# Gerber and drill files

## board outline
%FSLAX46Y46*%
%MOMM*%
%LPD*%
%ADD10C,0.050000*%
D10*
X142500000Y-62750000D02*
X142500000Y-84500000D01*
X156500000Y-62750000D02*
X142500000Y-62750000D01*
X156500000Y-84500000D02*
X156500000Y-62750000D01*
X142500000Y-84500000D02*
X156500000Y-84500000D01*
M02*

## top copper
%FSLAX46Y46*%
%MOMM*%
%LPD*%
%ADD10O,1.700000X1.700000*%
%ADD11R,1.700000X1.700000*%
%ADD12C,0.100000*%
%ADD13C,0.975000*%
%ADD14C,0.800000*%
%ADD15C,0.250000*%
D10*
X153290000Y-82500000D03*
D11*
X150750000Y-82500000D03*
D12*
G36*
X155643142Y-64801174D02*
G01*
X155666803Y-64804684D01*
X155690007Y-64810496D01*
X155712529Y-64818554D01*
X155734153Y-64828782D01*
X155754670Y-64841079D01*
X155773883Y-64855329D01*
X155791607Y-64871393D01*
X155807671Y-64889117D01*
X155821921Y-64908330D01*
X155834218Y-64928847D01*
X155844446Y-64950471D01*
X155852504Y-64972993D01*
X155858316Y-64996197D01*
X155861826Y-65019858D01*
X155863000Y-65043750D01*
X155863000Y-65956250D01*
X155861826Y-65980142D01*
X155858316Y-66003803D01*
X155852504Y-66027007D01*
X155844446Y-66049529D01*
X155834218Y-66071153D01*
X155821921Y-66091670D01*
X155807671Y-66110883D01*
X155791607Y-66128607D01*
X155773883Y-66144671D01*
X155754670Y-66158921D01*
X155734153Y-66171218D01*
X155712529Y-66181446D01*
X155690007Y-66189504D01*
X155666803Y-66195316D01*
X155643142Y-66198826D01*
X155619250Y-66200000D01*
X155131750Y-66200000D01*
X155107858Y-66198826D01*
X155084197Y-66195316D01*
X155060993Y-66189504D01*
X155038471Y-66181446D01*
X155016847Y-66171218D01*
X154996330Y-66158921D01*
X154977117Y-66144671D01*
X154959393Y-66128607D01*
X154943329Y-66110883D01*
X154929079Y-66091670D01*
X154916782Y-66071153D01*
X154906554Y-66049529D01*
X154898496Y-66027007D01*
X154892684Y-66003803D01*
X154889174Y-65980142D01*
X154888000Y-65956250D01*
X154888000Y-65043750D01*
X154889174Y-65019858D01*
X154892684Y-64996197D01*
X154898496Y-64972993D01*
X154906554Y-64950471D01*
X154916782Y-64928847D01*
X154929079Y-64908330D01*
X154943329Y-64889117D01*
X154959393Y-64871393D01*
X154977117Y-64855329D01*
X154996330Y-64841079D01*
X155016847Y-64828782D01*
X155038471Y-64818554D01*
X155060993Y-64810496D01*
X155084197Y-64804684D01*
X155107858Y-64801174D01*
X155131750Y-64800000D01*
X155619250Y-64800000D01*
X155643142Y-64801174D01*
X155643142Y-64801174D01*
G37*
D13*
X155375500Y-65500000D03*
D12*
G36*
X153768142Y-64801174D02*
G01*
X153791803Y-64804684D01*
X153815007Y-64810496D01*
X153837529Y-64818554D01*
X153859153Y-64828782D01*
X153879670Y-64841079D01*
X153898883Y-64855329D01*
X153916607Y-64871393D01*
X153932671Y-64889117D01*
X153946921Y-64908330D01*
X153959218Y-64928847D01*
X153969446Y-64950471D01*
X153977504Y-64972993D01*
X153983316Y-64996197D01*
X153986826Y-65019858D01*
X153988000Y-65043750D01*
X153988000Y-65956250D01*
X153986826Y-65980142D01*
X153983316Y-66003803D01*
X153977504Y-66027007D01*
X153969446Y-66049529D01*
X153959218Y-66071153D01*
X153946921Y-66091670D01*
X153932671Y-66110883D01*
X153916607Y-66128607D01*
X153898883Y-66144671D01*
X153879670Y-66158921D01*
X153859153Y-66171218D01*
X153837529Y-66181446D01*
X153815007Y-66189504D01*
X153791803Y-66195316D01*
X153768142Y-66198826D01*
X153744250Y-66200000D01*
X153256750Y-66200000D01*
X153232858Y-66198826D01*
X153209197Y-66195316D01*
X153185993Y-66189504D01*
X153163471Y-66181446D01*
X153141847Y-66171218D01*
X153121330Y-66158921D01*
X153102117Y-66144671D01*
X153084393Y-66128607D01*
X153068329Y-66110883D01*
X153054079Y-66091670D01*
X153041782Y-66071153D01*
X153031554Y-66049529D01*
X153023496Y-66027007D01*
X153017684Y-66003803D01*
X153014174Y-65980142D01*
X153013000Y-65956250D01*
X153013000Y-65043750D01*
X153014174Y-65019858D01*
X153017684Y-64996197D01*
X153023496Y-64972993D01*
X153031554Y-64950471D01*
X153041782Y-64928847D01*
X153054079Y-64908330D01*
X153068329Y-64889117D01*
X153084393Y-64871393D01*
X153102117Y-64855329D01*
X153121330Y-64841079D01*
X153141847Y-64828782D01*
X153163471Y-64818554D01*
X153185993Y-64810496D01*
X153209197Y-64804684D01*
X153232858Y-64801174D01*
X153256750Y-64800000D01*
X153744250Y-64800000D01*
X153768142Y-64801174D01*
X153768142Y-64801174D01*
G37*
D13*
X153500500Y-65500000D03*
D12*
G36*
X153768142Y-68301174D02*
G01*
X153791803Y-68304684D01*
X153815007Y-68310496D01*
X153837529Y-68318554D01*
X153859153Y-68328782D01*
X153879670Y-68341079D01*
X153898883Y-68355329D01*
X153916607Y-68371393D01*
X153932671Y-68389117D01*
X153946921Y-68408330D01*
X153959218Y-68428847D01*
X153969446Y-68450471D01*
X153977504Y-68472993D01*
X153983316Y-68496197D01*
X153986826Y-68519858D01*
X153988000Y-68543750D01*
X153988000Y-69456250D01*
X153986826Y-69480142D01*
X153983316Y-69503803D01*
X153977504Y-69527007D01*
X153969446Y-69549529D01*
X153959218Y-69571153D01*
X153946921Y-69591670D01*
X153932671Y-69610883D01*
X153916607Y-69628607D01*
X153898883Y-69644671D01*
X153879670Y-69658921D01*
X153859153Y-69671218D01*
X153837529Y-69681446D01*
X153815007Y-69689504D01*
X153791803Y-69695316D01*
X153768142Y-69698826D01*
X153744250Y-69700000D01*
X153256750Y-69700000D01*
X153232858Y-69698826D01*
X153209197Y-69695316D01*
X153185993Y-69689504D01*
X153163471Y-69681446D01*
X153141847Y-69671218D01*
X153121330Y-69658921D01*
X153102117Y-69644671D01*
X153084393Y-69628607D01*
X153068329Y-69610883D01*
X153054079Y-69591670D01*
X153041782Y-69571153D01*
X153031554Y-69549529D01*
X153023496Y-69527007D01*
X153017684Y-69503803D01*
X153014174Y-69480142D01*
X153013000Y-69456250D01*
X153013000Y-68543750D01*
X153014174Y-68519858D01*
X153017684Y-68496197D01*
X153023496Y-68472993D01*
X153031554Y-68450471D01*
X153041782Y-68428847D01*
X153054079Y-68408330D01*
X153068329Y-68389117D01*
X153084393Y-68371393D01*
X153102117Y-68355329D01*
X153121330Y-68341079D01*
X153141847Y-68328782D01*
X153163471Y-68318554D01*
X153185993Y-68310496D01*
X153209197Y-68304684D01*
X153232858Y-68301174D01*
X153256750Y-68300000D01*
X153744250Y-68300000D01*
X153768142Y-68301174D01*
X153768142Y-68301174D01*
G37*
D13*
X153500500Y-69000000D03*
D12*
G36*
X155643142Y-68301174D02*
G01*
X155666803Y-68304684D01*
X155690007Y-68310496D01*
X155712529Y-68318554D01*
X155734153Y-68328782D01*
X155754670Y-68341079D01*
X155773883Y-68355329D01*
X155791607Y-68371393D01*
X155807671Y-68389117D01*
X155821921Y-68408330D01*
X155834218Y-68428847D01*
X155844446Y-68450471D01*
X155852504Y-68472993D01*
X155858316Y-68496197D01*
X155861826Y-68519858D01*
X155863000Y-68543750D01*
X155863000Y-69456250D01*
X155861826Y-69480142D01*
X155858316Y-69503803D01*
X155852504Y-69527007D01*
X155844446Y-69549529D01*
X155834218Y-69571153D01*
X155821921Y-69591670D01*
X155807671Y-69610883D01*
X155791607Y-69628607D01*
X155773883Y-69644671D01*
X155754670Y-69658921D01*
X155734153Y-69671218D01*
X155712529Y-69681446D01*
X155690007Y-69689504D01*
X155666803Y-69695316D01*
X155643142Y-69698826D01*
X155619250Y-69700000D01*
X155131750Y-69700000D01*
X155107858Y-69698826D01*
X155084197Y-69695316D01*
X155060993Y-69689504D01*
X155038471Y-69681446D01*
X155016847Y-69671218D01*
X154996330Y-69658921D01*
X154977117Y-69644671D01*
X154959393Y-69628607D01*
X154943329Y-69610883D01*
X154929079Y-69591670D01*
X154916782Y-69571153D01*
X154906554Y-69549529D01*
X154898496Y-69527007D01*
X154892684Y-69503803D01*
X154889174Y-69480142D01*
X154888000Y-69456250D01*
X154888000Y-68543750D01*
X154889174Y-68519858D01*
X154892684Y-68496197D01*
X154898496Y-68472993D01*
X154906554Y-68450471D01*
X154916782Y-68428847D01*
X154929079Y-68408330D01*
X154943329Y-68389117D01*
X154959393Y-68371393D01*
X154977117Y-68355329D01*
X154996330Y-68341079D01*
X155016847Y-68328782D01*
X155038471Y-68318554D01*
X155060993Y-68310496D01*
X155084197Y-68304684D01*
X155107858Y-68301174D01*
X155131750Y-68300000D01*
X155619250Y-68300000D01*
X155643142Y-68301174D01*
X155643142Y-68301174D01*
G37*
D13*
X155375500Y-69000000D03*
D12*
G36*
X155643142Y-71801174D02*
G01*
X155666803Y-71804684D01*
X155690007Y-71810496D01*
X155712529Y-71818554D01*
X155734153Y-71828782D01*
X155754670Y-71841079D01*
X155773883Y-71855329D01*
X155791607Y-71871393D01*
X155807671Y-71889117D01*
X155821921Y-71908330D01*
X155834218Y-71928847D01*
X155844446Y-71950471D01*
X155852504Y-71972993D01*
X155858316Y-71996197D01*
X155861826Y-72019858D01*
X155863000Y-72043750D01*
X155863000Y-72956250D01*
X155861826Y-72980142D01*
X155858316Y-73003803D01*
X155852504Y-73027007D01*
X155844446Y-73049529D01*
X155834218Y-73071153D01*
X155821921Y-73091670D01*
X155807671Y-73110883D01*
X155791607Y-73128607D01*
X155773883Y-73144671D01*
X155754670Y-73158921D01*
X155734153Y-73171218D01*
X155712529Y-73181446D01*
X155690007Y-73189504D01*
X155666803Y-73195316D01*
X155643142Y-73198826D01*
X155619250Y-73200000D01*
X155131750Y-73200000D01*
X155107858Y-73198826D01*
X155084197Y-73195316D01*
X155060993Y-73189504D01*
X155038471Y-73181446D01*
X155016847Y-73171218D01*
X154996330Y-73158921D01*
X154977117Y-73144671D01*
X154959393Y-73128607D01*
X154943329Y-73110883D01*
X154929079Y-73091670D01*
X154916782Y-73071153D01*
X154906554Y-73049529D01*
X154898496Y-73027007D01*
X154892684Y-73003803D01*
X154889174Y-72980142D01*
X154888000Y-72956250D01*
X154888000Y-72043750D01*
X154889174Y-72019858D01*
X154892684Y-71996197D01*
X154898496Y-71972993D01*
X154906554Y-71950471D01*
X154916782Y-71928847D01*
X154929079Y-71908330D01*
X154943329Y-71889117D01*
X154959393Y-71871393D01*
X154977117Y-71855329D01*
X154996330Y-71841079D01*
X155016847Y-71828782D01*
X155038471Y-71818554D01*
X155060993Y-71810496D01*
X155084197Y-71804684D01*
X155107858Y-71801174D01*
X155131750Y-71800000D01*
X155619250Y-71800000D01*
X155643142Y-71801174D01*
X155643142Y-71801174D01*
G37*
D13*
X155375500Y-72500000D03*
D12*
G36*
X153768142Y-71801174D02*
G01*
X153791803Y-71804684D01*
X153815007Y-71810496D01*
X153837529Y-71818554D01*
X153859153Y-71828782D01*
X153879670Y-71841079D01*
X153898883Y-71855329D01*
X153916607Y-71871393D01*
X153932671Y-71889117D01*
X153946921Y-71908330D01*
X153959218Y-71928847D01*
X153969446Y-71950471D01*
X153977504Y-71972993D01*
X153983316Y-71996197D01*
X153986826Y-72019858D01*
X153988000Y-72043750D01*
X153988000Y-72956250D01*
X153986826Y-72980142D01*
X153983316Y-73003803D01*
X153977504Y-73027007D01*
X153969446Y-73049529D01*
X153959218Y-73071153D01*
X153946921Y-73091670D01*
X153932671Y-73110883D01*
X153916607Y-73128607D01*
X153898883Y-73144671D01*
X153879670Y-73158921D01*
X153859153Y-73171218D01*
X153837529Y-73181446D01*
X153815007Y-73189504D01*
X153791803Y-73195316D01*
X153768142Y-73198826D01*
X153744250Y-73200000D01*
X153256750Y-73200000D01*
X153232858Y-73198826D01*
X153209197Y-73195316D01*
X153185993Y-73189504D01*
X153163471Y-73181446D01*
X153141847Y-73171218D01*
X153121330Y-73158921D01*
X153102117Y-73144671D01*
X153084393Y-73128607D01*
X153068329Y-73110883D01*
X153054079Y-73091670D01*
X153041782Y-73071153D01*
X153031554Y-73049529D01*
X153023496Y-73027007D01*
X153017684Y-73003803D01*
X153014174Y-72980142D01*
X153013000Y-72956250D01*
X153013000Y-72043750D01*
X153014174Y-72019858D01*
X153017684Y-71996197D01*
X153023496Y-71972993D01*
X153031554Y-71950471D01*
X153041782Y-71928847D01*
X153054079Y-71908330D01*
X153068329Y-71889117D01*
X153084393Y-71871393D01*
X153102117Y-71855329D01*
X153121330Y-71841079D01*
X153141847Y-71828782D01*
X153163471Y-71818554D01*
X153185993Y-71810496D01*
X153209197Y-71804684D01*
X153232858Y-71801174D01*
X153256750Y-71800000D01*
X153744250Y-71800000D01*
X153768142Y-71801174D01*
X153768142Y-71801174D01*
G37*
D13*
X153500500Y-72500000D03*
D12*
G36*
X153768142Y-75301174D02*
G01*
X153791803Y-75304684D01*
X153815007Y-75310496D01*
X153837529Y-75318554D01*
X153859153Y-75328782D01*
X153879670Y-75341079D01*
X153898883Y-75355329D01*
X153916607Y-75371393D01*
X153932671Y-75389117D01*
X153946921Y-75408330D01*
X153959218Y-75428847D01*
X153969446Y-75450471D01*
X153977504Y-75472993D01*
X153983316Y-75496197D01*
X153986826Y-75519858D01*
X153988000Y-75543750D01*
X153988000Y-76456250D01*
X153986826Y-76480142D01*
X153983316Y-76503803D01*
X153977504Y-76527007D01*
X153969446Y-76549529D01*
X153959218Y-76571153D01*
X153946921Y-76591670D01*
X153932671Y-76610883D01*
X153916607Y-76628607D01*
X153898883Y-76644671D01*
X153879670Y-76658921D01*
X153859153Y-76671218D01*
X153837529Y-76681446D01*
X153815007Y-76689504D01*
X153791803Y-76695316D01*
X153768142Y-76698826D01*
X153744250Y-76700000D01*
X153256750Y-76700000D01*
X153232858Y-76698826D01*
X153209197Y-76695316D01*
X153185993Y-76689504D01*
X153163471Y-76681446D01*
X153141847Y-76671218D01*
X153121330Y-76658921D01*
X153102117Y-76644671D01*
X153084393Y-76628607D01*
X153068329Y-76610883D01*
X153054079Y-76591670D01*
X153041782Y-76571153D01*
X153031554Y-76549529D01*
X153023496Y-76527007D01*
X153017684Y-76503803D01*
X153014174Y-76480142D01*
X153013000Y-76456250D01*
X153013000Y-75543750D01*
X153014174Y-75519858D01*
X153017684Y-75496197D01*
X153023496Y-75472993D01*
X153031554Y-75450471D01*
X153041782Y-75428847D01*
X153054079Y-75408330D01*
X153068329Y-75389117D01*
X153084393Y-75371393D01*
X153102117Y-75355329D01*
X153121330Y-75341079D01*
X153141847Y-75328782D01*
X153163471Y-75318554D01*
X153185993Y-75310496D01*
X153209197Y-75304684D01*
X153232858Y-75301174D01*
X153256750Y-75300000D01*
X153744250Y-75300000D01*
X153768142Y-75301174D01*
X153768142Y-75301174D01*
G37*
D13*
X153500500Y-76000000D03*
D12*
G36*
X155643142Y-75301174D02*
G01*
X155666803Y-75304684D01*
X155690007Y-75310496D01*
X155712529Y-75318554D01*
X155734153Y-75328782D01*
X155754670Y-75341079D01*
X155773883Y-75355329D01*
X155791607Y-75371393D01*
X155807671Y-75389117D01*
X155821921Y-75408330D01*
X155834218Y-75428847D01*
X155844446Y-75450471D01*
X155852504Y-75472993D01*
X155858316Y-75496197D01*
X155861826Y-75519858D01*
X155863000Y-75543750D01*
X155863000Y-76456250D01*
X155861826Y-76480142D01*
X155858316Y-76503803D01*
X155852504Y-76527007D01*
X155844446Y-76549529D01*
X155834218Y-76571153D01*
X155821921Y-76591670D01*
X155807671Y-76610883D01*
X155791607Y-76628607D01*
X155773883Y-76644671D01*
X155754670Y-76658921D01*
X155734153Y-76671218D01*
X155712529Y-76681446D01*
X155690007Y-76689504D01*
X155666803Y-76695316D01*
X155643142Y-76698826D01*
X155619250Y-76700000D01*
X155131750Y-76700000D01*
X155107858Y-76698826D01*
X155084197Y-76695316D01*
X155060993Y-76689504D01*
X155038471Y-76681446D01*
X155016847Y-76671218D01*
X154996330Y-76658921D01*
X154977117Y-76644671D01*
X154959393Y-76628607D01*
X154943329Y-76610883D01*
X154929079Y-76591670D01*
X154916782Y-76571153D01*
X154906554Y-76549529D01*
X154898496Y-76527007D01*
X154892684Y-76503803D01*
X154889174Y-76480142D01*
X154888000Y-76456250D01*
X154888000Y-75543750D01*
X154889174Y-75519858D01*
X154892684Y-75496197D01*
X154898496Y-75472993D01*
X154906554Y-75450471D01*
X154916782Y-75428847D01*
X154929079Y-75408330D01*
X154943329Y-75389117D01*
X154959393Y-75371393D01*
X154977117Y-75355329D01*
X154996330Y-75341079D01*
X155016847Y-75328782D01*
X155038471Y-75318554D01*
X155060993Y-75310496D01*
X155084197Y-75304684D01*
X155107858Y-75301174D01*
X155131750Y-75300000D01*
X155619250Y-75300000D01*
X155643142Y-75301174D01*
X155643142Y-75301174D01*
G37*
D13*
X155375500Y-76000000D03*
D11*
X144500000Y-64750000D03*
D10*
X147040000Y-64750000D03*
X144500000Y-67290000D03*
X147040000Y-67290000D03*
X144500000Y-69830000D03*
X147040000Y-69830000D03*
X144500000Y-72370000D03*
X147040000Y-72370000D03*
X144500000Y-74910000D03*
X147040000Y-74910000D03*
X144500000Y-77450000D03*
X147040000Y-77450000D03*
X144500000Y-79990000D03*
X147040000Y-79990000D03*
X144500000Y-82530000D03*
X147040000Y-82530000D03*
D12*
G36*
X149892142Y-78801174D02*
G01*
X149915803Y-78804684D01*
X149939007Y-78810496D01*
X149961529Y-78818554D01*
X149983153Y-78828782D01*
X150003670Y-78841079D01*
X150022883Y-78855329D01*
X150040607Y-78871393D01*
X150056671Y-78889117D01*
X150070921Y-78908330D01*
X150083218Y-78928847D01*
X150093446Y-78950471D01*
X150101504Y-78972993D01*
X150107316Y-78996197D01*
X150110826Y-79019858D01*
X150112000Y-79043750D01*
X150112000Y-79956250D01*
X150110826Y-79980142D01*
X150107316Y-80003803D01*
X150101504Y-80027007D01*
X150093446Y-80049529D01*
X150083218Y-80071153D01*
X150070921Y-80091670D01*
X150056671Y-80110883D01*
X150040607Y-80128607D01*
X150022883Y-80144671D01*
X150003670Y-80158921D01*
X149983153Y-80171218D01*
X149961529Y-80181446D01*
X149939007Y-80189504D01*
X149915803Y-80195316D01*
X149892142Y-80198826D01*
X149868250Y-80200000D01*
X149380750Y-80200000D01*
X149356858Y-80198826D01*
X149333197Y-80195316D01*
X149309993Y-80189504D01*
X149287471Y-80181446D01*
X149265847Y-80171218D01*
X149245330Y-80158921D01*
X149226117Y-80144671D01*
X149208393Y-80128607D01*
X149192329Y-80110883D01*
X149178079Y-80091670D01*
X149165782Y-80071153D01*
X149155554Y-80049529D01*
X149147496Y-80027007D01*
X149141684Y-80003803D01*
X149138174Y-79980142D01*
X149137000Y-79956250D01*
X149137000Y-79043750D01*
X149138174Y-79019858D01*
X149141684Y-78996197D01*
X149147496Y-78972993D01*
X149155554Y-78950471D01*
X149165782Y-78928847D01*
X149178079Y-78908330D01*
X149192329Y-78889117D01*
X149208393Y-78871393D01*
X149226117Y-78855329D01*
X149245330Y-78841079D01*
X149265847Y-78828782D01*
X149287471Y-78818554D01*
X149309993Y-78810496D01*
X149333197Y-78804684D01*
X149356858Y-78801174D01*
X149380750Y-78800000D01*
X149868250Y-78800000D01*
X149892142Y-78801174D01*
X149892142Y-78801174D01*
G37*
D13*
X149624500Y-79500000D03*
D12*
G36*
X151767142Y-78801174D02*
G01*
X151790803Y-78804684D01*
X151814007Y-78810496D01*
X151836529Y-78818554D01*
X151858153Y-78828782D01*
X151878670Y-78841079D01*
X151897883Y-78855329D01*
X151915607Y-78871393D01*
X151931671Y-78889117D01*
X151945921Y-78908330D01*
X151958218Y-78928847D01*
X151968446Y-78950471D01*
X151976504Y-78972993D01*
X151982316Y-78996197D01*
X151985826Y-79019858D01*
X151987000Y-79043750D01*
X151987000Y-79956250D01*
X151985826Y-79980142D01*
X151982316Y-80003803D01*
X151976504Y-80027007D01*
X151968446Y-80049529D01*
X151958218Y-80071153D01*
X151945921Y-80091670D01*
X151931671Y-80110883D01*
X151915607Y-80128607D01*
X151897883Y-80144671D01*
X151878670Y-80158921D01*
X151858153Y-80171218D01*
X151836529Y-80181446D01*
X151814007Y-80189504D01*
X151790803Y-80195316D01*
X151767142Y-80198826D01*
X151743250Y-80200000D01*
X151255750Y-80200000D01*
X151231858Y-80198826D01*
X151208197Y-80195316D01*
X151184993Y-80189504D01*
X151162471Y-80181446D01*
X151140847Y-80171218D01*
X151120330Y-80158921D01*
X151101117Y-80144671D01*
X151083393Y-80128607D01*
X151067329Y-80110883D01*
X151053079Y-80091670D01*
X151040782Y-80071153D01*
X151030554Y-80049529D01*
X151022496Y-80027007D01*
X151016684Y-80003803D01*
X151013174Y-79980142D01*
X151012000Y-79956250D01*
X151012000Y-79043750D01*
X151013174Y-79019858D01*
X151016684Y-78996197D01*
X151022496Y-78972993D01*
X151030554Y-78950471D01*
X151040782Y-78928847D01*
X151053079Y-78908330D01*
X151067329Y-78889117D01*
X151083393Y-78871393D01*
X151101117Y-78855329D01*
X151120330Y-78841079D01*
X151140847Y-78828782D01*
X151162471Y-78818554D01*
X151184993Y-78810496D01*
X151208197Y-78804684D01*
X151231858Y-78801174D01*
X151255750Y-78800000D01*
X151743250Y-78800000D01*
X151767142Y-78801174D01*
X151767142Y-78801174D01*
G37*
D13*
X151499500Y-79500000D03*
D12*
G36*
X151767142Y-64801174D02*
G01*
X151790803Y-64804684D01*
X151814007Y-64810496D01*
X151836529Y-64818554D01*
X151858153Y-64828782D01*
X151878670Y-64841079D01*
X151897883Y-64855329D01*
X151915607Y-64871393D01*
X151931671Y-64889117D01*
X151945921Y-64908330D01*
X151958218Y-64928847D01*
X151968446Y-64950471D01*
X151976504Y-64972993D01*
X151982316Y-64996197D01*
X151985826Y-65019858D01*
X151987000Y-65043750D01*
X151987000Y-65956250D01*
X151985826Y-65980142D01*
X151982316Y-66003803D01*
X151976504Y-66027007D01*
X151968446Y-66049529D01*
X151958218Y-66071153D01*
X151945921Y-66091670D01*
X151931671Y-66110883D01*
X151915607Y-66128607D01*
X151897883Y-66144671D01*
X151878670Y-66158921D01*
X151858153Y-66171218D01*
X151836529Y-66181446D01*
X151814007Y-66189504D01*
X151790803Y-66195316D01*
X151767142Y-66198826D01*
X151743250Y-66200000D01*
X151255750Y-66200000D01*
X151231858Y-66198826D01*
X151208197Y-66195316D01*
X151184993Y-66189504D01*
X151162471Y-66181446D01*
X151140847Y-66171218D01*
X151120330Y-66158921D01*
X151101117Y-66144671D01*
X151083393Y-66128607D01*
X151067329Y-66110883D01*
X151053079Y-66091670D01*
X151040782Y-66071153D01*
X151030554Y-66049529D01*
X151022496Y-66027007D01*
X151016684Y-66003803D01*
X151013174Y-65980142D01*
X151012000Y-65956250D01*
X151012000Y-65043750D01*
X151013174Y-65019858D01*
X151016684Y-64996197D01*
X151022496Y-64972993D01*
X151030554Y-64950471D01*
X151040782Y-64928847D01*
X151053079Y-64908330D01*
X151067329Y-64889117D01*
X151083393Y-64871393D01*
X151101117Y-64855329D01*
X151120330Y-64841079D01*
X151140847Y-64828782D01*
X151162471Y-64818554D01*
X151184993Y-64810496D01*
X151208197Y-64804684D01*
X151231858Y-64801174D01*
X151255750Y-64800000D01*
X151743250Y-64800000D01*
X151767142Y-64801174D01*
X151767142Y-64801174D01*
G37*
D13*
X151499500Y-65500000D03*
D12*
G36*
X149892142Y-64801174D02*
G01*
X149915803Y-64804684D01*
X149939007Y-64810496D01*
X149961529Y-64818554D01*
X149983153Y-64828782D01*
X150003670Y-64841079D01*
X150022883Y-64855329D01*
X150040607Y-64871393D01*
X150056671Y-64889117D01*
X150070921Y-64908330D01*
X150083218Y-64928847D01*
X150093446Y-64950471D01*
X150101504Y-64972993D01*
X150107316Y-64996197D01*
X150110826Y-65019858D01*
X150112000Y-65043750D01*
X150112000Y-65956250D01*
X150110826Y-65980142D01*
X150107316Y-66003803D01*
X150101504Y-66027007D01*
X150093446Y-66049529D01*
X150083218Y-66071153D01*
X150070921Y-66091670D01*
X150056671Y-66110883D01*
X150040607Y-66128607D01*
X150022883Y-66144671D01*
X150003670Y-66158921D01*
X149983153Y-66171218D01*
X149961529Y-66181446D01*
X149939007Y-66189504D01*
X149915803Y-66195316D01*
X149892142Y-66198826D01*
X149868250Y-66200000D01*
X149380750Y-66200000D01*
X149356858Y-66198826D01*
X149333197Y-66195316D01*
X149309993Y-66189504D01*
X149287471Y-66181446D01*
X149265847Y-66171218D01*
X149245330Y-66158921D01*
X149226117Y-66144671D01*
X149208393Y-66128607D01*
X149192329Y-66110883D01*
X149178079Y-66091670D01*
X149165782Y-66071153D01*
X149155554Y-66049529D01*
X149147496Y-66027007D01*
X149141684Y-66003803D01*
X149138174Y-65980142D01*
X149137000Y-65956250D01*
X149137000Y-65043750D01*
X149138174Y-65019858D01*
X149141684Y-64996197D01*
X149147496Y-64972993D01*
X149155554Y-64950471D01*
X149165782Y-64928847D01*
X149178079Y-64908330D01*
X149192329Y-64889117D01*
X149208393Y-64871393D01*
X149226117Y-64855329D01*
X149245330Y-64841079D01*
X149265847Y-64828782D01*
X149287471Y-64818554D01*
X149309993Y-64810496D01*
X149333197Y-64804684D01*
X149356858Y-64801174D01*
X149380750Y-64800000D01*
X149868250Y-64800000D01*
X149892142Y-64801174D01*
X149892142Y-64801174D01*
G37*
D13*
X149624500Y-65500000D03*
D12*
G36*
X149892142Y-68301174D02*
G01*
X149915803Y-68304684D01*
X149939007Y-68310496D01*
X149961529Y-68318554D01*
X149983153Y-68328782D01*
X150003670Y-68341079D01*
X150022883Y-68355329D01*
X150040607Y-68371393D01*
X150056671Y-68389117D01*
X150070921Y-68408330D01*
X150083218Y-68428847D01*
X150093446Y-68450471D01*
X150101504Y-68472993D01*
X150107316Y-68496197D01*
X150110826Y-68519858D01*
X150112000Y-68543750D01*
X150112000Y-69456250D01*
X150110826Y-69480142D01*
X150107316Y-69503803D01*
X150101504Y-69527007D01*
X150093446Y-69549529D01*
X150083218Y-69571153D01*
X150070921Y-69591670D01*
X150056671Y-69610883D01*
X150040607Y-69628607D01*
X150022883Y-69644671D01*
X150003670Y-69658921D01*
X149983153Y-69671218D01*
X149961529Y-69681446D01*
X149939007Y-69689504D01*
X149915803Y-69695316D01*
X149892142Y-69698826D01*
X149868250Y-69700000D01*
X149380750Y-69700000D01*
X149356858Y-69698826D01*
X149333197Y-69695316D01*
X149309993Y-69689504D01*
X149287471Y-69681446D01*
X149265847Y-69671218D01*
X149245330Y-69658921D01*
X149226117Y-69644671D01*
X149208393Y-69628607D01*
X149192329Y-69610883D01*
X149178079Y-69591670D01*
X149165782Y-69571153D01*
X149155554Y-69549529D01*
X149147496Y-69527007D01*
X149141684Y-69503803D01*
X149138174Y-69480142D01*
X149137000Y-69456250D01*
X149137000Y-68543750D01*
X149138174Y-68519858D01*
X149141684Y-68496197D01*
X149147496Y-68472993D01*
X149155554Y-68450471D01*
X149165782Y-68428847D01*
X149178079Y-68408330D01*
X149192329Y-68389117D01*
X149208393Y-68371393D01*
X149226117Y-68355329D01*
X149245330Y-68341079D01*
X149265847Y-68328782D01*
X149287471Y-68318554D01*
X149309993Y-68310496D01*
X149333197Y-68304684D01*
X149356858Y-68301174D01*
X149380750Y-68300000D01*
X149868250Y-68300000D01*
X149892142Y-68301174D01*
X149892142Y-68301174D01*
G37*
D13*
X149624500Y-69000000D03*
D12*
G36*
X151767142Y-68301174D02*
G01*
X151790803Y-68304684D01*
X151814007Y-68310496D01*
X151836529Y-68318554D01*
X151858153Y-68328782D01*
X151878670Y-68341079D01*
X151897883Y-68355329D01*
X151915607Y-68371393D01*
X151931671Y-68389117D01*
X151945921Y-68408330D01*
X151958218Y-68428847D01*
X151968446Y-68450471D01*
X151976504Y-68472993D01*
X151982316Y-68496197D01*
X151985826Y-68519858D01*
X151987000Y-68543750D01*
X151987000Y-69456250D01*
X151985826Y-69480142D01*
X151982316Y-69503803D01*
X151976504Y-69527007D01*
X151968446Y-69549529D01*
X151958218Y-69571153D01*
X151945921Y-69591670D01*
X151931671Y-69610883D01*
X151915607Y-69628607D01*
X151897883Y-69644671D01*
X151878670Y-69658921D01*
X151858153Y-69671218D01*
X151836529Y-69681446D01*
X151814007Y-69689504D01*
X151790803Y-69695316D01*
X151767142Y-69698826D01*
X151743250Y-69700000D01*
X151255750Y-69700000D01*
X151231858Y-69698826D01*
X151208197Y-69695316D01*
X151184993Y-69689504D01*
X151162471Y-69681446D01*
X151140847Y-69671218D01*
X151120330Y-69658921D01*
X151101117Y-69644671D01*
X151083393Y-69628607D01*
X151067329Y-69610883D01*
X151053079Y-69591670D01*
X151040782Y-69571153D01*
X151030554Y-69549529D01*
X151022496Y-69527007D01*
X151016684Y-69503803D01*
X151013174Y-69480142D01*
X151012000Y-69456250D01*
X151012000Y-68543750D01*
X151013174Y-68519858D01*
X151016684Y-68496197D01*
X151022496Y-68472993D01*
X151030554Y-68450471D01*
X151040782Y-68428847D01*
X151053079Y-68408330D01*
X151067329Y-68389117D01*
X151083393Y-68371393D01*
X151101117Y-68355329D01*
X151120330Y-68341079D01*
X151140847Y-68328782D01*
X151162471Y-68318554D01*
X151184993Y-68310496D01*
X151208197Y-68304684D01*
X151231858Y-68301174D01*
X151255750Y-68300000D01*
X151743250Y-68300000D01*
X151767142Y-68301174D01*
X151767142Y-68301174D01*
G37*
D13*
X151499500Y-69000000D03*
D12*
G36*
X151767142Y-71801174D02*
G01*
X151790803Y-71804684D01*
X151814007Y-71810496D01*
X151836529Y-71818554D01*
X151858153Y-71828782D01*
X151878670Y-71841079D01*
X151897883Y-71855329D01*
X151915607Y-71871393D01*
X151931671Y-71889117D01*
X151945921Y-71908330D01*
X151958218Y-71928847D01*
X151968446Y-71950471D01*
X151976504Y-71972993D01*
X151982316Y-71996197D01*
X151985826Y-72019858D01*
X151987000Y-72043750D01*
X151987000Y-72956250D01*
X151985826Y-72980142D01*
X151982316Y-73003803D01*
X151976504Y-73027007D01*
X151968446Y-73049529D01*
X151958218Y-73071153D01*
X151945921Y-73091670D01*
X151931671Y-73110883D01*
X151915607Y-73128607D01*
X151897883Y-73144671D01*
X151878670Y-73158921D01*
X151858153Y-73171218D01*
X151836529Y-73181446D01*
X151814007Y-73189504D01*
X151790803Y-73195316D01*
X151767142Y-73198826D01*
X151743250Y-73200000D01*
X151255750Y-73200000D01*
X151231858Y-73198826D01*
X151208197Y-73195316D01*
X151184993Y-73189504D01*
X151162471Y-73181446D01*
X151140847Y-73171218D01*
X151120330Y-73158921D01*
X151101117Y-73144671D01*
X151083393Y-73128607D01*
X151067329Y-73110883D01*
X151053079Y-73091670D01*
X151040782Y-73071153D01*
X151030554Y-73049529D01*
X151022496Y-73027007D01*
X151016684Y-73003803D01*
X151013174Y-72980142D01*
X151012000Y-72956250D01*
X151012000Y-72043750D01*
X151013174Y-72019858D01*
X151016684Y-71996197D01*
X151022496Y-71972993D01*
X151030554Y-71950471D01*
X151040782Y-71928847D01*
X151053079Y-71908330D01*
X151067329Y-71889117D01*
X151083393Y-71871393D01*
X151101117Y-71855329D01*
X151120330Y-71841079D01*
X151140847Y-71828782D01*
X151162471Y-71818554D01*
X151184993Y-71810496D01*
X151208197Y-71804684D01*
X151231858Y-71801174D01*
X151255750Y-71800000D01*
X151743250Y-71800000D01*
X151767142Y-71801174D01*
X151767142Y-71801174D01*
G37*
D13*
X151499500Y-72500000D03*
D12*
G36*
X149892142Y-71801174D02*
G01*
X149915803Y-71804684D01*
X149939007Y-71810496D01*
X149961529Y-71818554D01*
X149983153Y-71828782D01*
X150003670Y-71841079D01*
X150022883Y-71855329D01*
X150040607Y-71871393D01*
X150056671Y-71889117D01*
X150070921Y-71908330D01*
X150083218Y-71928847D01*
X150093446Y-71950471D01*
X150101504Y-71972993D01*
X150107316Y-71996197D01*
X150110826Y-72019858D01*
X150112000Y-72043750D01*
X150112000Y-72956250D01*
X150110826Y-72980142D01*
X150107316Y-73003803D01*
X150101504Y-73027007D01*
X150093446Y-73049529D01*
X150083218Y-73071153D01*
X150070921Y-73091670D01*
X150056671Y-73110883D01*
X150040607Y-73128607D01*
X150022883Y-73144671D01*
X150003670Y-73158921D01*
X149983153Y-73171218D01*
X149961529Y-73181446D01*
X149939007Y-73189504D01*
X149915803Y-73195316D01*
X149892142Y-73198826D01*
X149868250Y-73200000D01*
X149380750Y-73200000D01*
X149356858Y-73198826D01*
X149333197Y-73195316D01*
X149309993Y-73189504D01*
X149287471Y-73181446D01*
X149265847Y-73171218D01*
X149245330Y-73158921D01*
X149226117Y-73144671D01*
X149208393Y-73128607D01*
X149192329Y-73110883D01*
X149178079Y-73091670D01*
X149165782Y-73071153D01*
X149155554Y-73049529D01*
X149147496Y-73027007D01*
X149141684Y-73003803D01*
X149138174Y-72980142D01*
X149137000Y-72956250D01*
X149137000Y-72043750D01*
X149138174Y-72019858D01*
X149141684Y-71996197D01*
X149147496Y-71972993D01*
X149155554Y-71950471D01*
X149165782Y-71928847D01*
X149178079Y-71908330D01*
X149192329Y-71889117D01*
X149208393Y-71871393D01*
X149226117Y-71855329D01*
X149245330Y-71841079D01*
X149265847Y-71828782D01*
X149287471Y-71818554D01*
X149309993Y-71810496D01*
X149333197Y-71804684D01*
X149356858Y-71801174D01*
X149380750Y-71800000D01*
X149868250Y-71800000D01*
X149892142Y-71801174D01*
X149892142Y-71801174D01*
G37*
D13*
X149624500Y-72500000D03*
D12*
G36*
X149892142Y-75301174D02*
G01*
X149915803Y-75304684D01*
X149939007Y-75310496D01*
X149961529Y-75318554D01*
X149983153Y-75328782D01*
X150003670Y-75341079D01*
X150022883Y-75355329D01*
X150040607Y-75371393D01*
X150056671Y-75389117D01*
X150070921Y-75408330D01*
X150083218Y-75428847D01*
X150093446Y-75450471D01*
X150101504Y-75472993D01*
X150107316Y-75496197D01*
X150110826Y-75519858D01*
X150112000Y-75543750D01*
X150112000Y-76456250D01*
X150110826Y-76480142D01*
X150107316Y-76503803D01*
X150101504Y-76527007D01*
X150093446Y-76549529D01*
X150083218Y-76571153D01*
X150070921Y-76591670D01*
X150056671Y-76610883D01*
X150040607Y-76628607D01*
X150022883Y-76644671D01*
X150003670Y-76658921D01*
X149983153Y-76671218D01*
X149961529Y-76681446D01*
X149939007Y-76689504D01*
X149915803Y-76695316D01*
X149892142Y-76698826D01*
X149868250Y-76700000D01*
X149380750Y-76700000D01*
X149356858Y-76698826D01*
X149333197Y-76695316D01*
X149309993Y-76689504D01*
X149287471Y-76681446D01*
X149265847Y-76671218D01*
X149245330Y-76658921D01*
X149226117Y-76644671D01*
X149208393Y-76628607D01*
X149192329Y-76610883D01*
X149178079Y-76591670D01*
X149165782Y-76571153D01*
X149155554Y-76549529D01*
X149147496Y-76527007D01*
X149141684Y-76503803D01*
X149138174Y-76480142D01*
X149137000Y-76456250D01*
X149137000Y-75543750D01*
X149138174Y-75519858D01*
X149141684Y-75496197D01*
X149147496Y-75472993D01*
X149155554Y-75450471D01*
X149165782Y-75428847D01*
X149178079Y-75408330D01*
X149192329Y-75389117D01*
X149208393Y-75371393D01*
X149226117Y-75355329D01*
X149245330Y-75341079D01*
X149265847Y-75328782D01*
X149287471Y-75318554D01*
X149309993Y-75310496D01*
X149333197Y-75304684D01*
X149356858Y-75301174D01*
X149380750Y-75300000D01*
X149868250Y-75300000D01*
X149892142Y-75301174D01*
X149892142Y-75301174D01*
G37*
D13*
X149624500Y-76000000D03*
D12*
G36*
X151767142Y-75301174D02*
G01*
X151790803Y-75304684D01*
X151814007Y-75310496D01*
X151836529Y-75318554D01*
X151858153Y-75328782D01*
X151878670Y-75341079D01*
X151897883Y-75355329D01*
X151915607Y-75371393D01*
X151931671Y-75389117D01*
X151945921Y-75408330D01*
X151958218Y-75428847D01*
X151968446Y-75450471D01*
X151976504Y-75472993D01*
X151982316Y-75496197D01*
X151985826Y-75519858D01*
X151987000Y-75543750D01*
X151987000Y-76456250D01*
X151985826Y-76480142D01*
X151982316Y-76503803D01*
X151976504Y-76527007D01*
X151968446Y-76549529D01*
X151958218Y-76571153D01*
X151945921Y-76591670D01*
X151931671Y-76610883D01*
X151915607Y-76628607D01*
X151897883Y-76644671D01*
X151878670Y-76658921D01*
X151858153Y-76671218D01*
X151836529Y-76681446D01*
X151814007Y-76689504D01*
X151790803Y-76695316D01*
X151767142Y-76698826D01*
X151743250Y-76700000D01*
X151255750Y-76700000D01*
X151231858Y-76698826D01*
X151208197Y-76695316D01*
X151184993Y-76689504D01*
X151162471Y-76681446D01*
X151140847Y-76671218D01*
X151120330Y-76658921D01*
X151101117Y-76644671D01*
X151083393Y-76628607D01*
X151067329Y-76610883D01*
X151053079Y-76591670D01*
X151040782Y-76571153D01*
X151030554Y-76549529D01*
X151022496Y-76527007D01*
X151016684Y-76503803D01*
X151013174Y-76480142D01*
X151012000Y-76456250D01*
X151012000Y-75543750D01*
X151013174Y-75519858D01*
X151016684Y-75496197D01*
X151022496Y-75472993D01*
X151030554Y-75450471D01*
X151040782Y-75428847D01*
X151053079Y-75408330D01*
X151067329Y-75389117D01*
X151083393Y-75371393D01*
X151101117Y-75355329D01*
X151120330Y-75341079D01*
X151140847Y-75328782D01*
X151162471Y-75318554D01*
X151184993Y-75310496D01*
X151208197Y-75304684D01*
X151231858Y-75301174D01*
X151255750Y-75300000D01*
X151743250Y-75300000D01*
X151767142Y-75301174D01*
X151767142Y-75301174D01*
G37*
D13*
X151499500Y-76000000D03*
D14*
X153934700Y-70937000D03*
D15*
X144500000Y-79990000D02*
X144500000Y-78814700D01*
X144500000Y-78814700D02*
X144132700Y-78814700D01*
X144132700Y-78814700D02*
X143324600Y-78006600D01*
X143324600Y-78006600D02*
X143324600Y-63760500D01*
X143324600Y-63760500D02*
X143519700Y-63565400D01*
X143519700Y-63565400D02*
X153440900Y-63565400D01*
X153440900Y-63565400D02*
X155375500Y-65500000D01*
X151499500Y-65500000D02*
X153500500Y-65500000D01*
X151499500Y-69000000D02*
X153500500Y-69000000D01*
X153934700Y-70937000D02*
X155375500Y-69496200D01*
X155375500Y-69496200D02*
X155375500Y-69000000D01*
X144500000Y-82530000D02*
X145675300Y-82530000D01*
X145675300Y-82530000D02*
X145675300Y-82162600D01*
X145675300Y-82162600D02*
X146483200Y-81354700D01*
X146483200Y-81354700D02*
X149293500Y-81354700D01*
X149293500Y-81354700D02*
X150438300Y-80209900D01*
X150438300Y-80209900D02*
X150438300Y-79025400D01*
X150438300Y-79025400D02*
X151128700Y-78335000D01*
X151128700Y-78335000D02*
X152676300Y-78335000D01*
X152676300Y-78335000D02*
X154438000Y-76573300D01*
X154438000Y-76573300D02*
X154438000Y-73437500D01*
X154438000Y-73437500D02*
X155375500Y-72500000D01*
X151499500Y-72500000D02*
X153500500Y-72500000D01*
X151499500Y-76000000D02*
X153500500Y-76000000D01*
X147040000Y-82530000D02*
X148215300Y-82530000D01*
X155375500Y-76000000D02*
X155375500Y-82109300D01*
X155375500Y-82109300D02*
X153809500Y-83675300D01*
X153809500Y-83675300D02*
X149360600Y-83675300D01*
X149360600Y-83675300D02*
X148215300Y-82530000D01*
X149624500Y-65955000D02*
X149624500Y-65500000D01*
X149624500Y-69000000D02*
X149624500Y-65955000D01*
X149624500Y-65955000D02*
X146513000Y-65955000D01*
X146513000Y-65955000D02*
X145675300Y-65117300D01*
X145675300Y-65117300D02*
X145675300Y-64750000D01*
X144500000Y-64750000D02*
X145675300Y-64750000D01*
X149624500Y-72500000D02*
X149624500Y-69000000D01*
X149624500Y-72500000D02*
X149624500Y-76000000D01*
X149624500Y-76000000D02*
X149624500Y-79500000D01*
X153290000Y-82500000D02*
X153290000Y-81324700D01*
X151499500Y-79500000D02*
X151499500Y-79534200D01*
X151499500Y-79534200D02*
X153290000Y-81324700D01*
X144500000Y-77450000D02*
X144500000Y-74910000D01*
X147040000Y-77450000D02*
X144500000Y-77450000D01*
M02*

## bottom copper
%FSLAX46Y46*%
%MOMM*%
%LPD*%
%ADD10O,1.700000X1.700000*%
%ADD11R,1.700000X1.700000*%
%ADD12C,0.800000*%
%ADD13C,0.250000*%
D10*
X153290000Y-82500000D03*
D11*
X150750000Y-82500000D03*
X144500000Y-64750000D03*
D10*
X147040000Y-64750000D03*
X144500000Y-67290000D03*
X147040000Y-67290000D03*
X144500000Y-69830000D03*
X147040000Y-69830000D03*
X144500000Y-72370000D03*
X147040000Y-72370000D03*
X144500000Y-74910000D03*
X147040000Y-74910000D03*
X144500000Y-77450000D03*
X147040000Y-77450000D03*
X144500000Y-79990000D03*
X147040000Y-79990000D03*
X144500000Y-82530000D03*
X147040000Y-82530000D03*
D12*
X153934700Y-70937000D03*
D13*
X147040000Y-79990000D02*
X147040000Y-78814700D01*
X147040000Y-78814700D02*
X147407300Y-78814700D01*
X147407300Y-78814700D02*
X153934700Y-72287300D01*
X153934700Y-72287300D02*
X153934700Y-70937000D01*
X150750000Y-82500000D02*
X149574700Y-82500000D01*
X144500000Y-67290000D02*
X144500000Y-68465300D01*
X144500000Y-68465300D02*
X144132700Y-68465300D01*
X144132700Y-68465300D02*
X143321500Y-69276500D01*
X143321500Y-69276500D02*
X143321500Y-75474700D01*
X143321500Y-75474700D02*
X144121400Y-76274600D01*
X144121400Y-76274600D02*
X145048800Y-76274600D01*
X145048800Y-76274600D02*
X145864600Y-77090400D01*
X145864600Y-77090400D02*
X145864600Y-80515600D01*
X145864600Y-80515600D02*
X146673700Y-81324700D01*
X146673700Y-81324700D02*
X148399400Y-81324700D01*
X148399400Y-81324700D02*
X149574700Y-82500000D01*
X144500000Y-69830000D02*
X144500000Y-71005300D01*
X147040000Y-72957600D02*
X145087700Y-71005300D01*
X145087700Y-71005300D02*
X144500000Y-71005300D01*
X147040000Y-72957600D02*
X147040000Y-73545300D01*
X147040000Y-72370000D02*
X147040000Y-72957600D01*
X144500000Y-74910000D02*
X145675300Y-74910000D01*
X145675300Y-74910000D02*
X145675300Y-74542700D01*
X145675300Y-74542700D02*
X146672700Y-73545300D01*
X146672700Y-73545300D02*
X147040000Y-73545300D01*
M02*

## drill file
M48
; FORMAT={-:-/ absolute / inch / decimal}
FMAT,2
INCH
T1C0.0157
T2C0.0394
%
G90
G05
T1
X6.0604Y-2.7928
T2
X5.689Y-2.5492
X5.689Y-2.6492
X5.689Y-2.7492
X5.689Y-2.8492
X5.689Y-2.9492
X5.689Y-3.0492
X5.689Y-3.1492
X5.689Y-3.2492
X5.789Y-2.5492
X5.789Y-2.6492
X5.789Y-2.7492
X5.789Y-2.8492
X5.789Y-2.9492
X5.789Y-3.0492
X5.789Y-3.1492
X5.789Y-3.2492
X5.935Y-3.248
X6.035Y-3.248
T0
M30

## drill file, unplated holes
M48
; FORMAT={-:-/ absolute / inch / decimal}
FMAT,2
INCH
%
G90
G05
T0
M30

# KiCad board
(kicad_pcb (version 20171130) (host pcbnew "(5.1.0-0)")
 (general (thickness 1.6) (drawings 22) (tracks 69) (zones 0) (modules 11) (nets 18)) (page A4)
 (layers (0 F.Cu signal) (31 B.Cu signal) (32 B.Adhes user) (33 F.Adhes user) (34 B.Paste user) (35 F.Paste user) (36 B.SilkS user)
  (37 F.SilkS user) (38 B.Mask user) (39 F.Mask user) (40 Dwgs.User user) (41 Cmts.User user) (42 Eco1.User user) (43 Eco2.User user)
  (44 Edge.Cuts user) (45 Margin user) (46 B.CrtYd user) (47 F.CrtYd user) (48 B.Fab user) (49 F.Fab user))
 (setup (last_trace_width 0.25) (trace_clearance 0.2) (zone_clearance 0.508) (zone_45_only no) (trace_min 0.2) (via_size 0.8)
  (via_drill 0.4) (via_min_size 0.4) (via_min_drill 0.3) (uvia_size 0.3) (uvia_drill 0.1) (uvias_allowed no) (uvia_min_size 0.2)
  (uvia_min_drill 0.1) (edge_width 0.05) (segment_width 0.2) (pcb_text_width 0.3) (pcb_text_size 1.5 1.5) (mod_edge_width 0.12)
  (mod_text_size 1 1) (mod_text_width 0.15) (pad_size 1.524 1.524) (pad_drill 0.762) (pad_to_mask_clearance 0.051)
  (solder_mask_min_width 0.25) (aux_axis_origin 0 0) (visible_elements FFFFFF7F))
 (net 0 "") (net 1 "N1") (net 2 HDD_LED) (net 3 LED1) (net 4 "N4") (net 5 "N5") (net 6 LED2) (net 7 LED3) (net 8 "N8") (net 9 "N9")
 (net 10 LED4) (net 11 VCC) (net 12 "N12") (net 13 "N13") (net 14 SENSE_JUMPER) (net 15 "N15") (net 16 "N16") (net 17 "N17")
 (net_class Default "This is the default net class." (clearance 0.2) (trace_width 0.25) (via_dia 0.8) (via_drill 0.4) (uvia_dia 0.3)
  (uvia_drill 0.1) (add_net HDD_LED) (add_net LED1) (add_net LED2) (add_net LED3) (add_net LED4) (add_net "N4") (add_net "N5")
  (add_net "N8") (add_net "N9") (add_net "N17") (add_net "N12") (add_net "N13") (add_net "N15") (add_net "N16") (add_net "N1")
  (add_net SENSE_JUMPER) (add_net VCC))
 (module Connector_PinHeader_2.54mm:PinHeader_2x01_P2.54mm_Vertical (layer F.Cu) (at 150.75 82.5)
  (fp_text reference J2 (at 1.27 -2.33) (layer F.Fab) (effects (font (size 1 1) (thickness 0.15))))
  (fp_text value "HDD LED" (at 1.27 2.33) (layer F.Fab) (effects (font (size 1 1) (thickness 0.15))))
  (pad 2 thru_hole oval (at 2.54 0) (size 1.7 1.7) (drill 1) (layers *.Cu *.Mask) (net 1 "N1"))
  (pad 1 thru_hole rect (at 0 0) (size 1.7 1.7) (drill 1) (layers *.Cu *.Mask) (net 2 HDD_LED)))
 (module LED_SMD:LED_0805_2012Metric (layer F.Cu) (at 154.438 65.5 180)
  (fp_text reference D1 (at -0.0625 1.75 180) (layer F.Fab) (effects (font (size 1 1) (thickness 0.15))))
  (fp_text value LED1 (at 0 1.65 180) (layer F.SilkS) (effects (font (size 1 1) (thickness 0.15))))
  (pad 1 smd roundrect (at -0.9375 0 180) (size 0.975 1.4) (layers F.Cu F.Paste F.Mask) (roundrect_rratio 0.25) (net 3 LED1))
  (pad 2 smd roundrect (at 0.9375 0 180) (size 0.975 1.4) (layers F.Cu F.Paste F.Mask) (roundrect_rratio 0.25) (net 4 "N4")))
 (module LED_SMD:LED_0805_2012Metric (layer F.Cu) (at 154.438 69 180)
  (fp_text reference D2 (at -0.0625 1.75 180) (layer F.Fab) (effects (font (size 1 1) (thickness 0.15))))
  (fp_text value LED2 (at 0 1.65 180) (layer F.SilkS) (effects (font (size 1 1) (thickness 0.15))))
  (pad 2 smd roundrect (at 0.9375 0 180) (size 0.975 1.4) (layers F.Cu F.Paste F.Mask) (roundrect_rratio 0.25) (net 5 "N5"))
  (pad 1 smd roundrect (at -0.9375 0 180) (size 0.975 1.4) (layers F.Cu F.Paste F.Mask) (roundrect_rratio 0.25) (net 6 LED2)))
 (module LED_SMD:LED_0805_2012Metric (layer F.Cu) (at 154.438 72.5 180)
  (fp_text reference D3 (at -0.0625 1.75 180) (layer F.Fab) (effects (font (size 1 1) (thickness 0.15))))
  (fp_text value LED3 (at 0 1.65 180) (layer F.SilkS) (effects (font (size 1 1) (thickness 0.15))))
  (pad 1 smd roundrect (at -0.9375 0 180) (size 0.975 1.4) (layers F.Cu F.Paste F.Mask) (roundrect_rratio 0.25) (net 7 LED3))
  (pad 2 smd roundrect (at 0.9375 0 180) (size 0.975 1.4) (layers F.Cu F.Paste F.Mask) (roundrect_rratio 0.25) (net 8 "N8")))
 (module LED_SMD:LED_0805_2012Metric (layer F.Cu) (at 154.438 76 180)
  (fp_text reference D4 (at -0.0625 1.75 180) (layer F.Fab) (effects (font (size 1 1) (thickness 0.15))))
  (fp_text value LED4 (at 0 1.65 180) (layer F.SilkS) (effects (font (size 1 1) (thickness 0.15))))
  (pad 2 smd roundrect (at 0.9375 0 180) (size 0.975 1.4) (layers F.Cu F.Paste F.Mask) (roundrect_rratio 0.25) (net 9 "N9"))
  (pad 1 smd roundrect (at -0.9375 0 180) (size 0.975 1.4) (layers F.Cu F.Paste F.Mask) (roundrect_rratio 0.25) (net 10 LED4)))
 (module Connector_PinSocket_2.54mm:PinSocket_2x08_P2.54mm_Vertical (layer B.Cu) (at 144.5 64.75 180)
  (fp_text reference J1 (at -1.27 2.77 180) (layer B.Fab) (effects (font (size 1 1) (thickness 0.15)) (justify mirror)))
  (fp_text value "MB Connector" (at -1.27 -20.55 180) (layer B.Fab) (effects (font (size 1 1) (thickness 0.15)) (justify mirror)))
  (pad 1 thru_hole rect (at 0 0 180) (size 1.7 1.7) (drill 1) (layers *.Cu *.Mask) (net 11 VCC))
  (pad 2 thru_hole oval (at -2.54 0 180) (size 1.7 1.7) (drill 1) (layers *.Cu *.Mask) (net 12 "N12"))
  (pad 3 thru_hole oval (at 0 -2.54 180) (size 1.7 1.7) (drill 1) (layers *.Cu *.Mask) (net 2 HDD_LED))
  (pad 4 thru_hole oval (at -2.54 -2.54 180) (size 1.7 1.7) (drill 1) (layers *.Cu *.Mask) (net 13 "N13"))
  (pad 5 thru_hole oval (at 0 -5.08 180) (size 1.7 1.7) (drill 1) (layers *.Cu *.Mask) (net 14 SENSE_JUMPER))
  (pad 6 thru_hole oval (at -2.54 -5.08 180) (size 1.7 1.7) (drill 1) (layers *.Cu *.Mask) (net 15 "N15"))
  (pad 7 thru_hole oval (at 0 -7.62 180) (size 1.7 1.7) (drill 1) (layers *.Cu *.Mask) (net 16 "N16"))
  (pad 8 thru_hole oval (at -2.54 -7.62 180) (size 1.7 1.7) (drill 1) (layers *.Cu *.Mask) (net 14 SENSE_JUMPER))
  (pad 9 thru_hole oval (at 0 -10.16 180) (size 1.7 1.7) (drill 1) (layers *.Cu *.Mask) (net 14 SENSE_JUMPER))
  (pad 10 thru_hole oval (at -2.54 -10.16 180) (size 1.7 1.7) (drill 1) (layers *.Cu *.Mask) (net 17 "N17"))
  (pad 11 thru_hole oval (at 0 -12.7 180) (size 1.7 1.7) (drill 1) (layers *.Cu *.Mask) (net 14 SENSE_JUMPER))
  (pad 12 thru_hole oval (at -2.54 -12.7 180) (size 1.7 1.7) (drill 1) (layers *.Cu *.Mask) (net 14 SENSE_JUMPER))
  (pad 13 thru_hole oval (at 0 -15.24 180) (size 1.7 1.7) (drill 1) (layers *.Cu *.Mask) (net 3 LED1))
  (pad 14 thru_hole oval (at -2.54 -15.24 180) (size 1.7 1.7) (drill 1) (layers *.Cu *.Mask) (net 6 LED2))
  (pad 15 thru_hole oval (at 0 -17.78 180) (size 1.7 1.7) (drill 1) (layers *.Cu *.Mask) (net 7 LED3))
  (pad 16 thru_hole oval (at -2.54 -17.78 180) (size 1.7 1.7) (drill 1) (layers *.Cu *.Mask) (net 10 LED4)))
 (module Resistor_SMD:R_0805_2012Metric (layer F.Cu) (at 150.562 79.5)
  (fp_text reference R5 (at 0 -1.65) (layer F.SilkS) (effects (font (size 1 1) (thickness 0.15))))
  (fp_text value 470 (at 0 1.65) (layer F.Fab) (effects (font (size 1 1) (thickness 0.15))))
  (pad 1 smd roundrect (at -0.9375 0) (size 0.975 1.4) (layers F.Cu F.Paste F.Mask) (roundrect_rratio 0.25) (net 11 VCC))
  (pad 2 smd roundrect (at 0.9375 0) (size 0.975 1.4) (layers F.Cu F.Paste F.Mask) (roundrect_rratio 0.25) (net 1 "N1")))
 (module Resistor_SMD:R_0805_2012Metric (layer F.Cu) (at 150.562 65.5)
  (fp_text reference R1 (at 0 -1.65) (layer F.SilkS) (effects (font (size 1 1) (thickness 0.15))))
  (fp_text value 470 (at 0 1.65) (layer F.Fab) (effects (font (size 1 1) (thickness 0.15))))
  (pad 2 smd roundrect (at 0.9375 0) (size 0.975 1.4) (layers F.Cu F.Paste F.Mask) (roundrect_rratio 0.25) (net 4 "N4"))
  (pad 1 smd roundrect (at -0.9375 0) (size 0.975 1.4) (layers F.Cu F.Paste F.Mask) (roundrect_rratio 0.25) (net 11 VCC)))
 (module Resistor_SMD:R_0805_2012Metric (layer F.Cu) (at 150.562 69)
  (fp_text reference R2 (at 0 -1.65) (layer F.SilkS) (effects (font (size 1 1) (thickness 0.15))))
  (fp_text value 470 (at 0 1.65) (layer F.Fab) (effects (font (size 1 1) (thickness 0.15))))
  (pad 1 smd roundrect (at -0.9375 0) (size 0.975 1.4) (layers F.Cu F.Paste F.Mask) (roundrect_rratio 0.25) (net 11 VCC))
  (pad 2 smd roundrect (at 0.9375 0) (size 0.975 1.4) (layers F.Cu F.Paste F.Mask) (roundrect_rratio 0.25) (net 5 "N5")))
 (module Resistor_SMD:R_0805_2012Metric (layer F.Cu) (at 150.562 72.5)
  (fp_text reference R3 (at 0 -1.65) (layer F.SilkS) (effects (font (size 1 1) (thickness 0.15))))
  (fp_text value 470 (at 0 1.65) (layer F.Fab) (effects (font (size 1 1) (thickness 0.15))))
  (pad 2 smd roundrect (at 0.9375 0) (size 0.975 1.4) (layers F.Cu F.Paste F.Mask) (roundrect_rratio 0.25) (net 8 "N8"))
  (pad 1 smd roundrect (at -0.9375 0) (size 0.975 1.4) (layers F.Cu F.Paste F.Mask) (roundrect_rratio 0.25) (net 11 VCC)))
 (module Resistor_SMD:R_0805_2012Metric (layer F.Cu) (at 150.562 76)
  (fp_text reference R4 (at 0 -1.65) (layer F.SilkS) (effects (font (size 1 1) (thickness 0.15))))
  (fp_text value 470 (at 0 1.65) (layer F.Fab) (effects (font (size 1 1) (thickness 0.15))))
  (pad 1 smd roundrect (at -0.9375 0) (size 0.975 1.4) (layers F.Cu F.Paste F.Mask) (roundrect_rratio 0.25) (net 11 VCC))
  (pad 2 smd roundrect (at 0.9375 0) (size 0.975 1.4) (layers F.Cu F.Paste F.Mask) (roundrect_rratio 0.25) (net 9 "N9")))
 (gr_line (start 142.5 62.75) (end 142.5 84.5) (layer Edge.Cuts) (width 0.05))
 (gr_line (start 156.5 62.75) (end 142.5 62.75) (layer Edge.Cuts) (width 0.05))
 (gr_line (start 156.5 84.5) (end 156.5 62.75) (layer Edge.Cuts) (width 0.05))
 (gr_line (start 142.5 84.5) (end 156.5 84.5) (layer Edge.Cuts) (width 0.05))
 (segment (start 144.5 79.99) (end 144.5 78.8147) (width 0.25) (layer F.Cu) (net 3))
 (segment (start 144.5 78.8147) (end 144.1327 78.8147) (width 0.25) (layer F.Cu) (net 3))
 (segment (start 144.1327 78.8147) (end 143.3246 78.0066) (width 0.25) (layer F.Cu) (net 3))
 (segment (start 143.3246 78.0066) (end 143.3246 63.7605) (width 0.25) (layer F.Cu) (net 3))
 (segment (start 143.3246 63.7605) (end 143.5197 63.5654) (width 0.25) (layer F.Cu) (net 3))
 (segment (start 143.5197 63.5654) (end 153.4409 63.5654) (width 0.25) (layer F.Cu) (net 3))
 (segment (start 153.4409 63.5654) (end 155.3755 65.5) (width 0.25) (layer F.Cu) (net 3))
 (segment (start 151.4995 65.5) (end 153.5005 65.5) (width 0.25) (layer F.Cu) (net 4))
 (segment (start 151.4995 69) (end 153.5005 69) (width 0.25) (layer F.Cu) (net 5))
 (segment (start 147.04 79.99) (end 147.04 78.8147) (width 0.25) (layer B.Cu) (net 6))
 (segment (start 153.9347 70.937) (end 155.3755 69.4962) (width 0.25) (layer F.Cu) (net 6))
 (segment (start 155.3755 69.4962) (end 155.3755 69) (width 0.25) (layer F.Cu) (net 6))
 (segment (start 147.04 78.8147) (end 147.4073 78.8147) (width 0.25) (layer B.Cu) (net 6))
 (segment (start 147.4073 78.8147) (end 153.9347 72.2873) (width 0.25) (layer B.Cu) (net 6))
 (segment (start 153.9347 72.2873) (end 153.9347 70.937) (width 0.25) (layer B.Cu) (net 6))
 (via (at 153.9347 70.937) (size 0.8) (layers F.Cu B.Cu) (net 6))
 (segment (start 144.5 82.53) (end 145.6753 82.53) (width 0.25) (layer F.Cu) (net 7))
 (segment (start 145.6753 82.53) (end 145.6753 82.1626) (width 0.25) (layer F.Cu) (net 7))
 (segment (start 145.6753 82.1626) (end 146.4832 81.3547) (width 0.25) (layer F.Cu) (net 7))
 (segment (start 146.4832 81.3547) (end 149.2935 81.3547) (width 0.25) (layer F.Cu) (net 7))
 (segment (start 149.2935 81.3547) (end 150.4383 80.2099) (width 0.25) (layer F.Cu) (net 7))
 (segment (start 150.4383 80.2099) (end 150.4383 79.0254) (width 0.25) (layer F.Cu) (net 7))
 (segment (start 150.4383 79.0254) (end 151.1287 78.335) (width 0.25) (layer F.Cu) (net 7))
 (segment (start 151.1287 78.335) (end 152.6763 78.335) (width 0.25) (layer F.Cu) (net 7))
 (segment (start 152.6763 78.335) (end 154.438 76.5733) (width 0.25) (layer F.Cu) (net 7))
 (segment (start 154.438 76.5733) (end 154.438 73.4375) (width 0.25) (layer F.Cu) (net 7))
 (segment (start 154.438 73.4375) (end 155.3755 72.5) (width 0.25) (layer F.Cu) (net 7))
 (segment (start 151.4995 72.5) (end 153.5005 72.5) (width 0.25) (layer F.Cu) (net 8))
 (segment (start 151.4995 76) (end 153.5005 76) (width 0.25) (layer F.Cu) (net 9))
 (segment (start 147.04 82.53) (end 148.2153 82.53) (width 0.25) (layer F.Cu) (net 10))
 (segment (start 155.3755 76) (end 155.3755 82.1093) (width 0.25) (layer F.Cu) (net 10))
 (segment (start 155.3755 82.1093) (end 153.8095 83.6753) (width 0.25) (layer F.Cu) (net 10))
 (segment (start 153.8095 83.6753) (end 149.3606 83.6753) (width 0.25) (layer F.Cu) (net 10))
 (segment (start 149.3606 83.6753) (end 148.2153 82.53) (width 0.25) (layer F.Cu) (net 10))
 (segment (start 150.75 82.5) (end 149.5747 82.5) (width 0.25) (layer B.Cu) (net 2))
 (segment (start 144.5 67.29) (end 144.5 68.4653) (width 0.25) (layer B.Cu) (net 2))
 (segment (start 144.5 68.4653) (end 144.1327 68.4653) (width 0.25) (layer B.Cu) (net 2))
 (segment (start 144.1327 68.4653) (end 143.3215 69.2765) (width 0.25) (layer B.Cu) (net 2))
 (segment (start 143.3215 69.2765) (end 143.3215 75.4747) (width 0.25) (layer B.Cu) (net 2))
 (segment (start 143.3215 75.4747) (end 144.1214 76.2746) (width 0.25) (layer B.Cu) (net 2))
 (segment (start 144.1214 76.2746) (end 145.0488 76.2746) (width 0.25) (layer B.Cu) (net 2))
 (segment (start 145.0488 76.2746) (end 145.8646 77.0904) (width 0.25) (layer B.Cu) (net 2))
 (segment (start 145.8646 77.0904) (end 145.8646 80.5156) (width 0.25) (layer B.Cu) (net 2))
 (segment (start 145.8646 80.5156) (end 146.6737 81.3247) (width 0.25) (layer B.Cu) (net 2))
 (segment (start 146.6737 81.3247) (end 148.3994 81.3247) (width 0.25) (layer B.Cu) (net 2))
 (segment (start 148.3994 81.3247) (end 149.5747 82.5) (width 0.25) (layer B.Cu) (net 2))
 (segment (start 149.6245 65.955) (end 149.6245 65.5) (width 0.25) (layer F.Cu) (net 11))
 (segment (start 149.6245 69) (end 149.6245 65.955) (width 0.25) (layer F.Cu) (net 11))
 (segment (start 149.6245 65.955) (end 146.513 65.955) (width 0.25) (layer F.Cu) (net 11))
 (segment (start 146.513 65.955) (end 145.6753 65.1173) (width 0.25) (layer F.Cu) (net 11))
 (segment (start 145.6753 65.1173) (end 145.6753 64.75) (width 0.25) (layer F.Cu) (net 11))
 (segment (start 144.5 64.75) (end 145.6753 64.75) (width 0.25) (layer F.Cu) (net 11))
 (segment (start 149.6245 72.5) (end 149.6245 69) (width 0.25) (layer F.Cu) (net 11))
 (segment (start 149.6245 72.5) (end 149.6245 76) (width 0.25) (layer F.Cu) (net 11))
 (segment (start 149.6245 76) (end 149.6245 79.5) (width 0.25) (layer F.Cu) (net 11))
 (segment (start 153.29 82.5) (end 153.29 81.3247) (width 0.25) (layer F.Cu) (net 1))
 (segment (start 151.4995 79.5) (end 151.4995 79.5342) (width 0.25) (layer F.Cu) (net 1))
 (segment (start 151.4995 79.5342) (end 153.29 81.3247) (width 0.25) (layer F.Cu) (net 1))
 (segment (start 144.5 69.83) (end 144.5 71.0053) (width 0.25) (layer B.Cu) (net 14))
 (segment (start 147.04 72.9576) (end 145.0877 71.0053) (width 0.25) (layer B.Cu) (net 14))
 (segment (start 145.0877 71.0053) (end 144.5 71.0053) (width 0.25) (layer B.Cu) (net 14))
 (segment (start 147.04 72.9576) (end 147.04 73.5453) (width 0.25) (layer B.Cu) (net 14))
 (segment (start 147.04 72.37) (end 147.04 72.9576) (width 0.25) (layer B.Cu) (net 14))
 (segment (start 144.5 74.91) (end 145.6753 74.91) (width 0.25) (layer B.Cu) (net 14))
 (segment (start 145.6753 74.91) (end 145.6753 74.5427) (width 0.25) (layer B.Cu) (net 14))
 (segment (start 145.6753 74.5427) (end 146.6727 73.5453) (width 0.25) (layer B.Cu) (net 14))
 (segment (start 146.6727 73.5453) (end 147.04 73.5453) (width 0.25) (layer B.Cu) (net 14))
 (segment (start 144.5 77.45) (end 144.5 74.91) (width 0.25) (layer F.Cu) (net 14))
 (segment (start 147.04 77.45) (end 144.5 77.45) (width 0.25) (layer F.Cu) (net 14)))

